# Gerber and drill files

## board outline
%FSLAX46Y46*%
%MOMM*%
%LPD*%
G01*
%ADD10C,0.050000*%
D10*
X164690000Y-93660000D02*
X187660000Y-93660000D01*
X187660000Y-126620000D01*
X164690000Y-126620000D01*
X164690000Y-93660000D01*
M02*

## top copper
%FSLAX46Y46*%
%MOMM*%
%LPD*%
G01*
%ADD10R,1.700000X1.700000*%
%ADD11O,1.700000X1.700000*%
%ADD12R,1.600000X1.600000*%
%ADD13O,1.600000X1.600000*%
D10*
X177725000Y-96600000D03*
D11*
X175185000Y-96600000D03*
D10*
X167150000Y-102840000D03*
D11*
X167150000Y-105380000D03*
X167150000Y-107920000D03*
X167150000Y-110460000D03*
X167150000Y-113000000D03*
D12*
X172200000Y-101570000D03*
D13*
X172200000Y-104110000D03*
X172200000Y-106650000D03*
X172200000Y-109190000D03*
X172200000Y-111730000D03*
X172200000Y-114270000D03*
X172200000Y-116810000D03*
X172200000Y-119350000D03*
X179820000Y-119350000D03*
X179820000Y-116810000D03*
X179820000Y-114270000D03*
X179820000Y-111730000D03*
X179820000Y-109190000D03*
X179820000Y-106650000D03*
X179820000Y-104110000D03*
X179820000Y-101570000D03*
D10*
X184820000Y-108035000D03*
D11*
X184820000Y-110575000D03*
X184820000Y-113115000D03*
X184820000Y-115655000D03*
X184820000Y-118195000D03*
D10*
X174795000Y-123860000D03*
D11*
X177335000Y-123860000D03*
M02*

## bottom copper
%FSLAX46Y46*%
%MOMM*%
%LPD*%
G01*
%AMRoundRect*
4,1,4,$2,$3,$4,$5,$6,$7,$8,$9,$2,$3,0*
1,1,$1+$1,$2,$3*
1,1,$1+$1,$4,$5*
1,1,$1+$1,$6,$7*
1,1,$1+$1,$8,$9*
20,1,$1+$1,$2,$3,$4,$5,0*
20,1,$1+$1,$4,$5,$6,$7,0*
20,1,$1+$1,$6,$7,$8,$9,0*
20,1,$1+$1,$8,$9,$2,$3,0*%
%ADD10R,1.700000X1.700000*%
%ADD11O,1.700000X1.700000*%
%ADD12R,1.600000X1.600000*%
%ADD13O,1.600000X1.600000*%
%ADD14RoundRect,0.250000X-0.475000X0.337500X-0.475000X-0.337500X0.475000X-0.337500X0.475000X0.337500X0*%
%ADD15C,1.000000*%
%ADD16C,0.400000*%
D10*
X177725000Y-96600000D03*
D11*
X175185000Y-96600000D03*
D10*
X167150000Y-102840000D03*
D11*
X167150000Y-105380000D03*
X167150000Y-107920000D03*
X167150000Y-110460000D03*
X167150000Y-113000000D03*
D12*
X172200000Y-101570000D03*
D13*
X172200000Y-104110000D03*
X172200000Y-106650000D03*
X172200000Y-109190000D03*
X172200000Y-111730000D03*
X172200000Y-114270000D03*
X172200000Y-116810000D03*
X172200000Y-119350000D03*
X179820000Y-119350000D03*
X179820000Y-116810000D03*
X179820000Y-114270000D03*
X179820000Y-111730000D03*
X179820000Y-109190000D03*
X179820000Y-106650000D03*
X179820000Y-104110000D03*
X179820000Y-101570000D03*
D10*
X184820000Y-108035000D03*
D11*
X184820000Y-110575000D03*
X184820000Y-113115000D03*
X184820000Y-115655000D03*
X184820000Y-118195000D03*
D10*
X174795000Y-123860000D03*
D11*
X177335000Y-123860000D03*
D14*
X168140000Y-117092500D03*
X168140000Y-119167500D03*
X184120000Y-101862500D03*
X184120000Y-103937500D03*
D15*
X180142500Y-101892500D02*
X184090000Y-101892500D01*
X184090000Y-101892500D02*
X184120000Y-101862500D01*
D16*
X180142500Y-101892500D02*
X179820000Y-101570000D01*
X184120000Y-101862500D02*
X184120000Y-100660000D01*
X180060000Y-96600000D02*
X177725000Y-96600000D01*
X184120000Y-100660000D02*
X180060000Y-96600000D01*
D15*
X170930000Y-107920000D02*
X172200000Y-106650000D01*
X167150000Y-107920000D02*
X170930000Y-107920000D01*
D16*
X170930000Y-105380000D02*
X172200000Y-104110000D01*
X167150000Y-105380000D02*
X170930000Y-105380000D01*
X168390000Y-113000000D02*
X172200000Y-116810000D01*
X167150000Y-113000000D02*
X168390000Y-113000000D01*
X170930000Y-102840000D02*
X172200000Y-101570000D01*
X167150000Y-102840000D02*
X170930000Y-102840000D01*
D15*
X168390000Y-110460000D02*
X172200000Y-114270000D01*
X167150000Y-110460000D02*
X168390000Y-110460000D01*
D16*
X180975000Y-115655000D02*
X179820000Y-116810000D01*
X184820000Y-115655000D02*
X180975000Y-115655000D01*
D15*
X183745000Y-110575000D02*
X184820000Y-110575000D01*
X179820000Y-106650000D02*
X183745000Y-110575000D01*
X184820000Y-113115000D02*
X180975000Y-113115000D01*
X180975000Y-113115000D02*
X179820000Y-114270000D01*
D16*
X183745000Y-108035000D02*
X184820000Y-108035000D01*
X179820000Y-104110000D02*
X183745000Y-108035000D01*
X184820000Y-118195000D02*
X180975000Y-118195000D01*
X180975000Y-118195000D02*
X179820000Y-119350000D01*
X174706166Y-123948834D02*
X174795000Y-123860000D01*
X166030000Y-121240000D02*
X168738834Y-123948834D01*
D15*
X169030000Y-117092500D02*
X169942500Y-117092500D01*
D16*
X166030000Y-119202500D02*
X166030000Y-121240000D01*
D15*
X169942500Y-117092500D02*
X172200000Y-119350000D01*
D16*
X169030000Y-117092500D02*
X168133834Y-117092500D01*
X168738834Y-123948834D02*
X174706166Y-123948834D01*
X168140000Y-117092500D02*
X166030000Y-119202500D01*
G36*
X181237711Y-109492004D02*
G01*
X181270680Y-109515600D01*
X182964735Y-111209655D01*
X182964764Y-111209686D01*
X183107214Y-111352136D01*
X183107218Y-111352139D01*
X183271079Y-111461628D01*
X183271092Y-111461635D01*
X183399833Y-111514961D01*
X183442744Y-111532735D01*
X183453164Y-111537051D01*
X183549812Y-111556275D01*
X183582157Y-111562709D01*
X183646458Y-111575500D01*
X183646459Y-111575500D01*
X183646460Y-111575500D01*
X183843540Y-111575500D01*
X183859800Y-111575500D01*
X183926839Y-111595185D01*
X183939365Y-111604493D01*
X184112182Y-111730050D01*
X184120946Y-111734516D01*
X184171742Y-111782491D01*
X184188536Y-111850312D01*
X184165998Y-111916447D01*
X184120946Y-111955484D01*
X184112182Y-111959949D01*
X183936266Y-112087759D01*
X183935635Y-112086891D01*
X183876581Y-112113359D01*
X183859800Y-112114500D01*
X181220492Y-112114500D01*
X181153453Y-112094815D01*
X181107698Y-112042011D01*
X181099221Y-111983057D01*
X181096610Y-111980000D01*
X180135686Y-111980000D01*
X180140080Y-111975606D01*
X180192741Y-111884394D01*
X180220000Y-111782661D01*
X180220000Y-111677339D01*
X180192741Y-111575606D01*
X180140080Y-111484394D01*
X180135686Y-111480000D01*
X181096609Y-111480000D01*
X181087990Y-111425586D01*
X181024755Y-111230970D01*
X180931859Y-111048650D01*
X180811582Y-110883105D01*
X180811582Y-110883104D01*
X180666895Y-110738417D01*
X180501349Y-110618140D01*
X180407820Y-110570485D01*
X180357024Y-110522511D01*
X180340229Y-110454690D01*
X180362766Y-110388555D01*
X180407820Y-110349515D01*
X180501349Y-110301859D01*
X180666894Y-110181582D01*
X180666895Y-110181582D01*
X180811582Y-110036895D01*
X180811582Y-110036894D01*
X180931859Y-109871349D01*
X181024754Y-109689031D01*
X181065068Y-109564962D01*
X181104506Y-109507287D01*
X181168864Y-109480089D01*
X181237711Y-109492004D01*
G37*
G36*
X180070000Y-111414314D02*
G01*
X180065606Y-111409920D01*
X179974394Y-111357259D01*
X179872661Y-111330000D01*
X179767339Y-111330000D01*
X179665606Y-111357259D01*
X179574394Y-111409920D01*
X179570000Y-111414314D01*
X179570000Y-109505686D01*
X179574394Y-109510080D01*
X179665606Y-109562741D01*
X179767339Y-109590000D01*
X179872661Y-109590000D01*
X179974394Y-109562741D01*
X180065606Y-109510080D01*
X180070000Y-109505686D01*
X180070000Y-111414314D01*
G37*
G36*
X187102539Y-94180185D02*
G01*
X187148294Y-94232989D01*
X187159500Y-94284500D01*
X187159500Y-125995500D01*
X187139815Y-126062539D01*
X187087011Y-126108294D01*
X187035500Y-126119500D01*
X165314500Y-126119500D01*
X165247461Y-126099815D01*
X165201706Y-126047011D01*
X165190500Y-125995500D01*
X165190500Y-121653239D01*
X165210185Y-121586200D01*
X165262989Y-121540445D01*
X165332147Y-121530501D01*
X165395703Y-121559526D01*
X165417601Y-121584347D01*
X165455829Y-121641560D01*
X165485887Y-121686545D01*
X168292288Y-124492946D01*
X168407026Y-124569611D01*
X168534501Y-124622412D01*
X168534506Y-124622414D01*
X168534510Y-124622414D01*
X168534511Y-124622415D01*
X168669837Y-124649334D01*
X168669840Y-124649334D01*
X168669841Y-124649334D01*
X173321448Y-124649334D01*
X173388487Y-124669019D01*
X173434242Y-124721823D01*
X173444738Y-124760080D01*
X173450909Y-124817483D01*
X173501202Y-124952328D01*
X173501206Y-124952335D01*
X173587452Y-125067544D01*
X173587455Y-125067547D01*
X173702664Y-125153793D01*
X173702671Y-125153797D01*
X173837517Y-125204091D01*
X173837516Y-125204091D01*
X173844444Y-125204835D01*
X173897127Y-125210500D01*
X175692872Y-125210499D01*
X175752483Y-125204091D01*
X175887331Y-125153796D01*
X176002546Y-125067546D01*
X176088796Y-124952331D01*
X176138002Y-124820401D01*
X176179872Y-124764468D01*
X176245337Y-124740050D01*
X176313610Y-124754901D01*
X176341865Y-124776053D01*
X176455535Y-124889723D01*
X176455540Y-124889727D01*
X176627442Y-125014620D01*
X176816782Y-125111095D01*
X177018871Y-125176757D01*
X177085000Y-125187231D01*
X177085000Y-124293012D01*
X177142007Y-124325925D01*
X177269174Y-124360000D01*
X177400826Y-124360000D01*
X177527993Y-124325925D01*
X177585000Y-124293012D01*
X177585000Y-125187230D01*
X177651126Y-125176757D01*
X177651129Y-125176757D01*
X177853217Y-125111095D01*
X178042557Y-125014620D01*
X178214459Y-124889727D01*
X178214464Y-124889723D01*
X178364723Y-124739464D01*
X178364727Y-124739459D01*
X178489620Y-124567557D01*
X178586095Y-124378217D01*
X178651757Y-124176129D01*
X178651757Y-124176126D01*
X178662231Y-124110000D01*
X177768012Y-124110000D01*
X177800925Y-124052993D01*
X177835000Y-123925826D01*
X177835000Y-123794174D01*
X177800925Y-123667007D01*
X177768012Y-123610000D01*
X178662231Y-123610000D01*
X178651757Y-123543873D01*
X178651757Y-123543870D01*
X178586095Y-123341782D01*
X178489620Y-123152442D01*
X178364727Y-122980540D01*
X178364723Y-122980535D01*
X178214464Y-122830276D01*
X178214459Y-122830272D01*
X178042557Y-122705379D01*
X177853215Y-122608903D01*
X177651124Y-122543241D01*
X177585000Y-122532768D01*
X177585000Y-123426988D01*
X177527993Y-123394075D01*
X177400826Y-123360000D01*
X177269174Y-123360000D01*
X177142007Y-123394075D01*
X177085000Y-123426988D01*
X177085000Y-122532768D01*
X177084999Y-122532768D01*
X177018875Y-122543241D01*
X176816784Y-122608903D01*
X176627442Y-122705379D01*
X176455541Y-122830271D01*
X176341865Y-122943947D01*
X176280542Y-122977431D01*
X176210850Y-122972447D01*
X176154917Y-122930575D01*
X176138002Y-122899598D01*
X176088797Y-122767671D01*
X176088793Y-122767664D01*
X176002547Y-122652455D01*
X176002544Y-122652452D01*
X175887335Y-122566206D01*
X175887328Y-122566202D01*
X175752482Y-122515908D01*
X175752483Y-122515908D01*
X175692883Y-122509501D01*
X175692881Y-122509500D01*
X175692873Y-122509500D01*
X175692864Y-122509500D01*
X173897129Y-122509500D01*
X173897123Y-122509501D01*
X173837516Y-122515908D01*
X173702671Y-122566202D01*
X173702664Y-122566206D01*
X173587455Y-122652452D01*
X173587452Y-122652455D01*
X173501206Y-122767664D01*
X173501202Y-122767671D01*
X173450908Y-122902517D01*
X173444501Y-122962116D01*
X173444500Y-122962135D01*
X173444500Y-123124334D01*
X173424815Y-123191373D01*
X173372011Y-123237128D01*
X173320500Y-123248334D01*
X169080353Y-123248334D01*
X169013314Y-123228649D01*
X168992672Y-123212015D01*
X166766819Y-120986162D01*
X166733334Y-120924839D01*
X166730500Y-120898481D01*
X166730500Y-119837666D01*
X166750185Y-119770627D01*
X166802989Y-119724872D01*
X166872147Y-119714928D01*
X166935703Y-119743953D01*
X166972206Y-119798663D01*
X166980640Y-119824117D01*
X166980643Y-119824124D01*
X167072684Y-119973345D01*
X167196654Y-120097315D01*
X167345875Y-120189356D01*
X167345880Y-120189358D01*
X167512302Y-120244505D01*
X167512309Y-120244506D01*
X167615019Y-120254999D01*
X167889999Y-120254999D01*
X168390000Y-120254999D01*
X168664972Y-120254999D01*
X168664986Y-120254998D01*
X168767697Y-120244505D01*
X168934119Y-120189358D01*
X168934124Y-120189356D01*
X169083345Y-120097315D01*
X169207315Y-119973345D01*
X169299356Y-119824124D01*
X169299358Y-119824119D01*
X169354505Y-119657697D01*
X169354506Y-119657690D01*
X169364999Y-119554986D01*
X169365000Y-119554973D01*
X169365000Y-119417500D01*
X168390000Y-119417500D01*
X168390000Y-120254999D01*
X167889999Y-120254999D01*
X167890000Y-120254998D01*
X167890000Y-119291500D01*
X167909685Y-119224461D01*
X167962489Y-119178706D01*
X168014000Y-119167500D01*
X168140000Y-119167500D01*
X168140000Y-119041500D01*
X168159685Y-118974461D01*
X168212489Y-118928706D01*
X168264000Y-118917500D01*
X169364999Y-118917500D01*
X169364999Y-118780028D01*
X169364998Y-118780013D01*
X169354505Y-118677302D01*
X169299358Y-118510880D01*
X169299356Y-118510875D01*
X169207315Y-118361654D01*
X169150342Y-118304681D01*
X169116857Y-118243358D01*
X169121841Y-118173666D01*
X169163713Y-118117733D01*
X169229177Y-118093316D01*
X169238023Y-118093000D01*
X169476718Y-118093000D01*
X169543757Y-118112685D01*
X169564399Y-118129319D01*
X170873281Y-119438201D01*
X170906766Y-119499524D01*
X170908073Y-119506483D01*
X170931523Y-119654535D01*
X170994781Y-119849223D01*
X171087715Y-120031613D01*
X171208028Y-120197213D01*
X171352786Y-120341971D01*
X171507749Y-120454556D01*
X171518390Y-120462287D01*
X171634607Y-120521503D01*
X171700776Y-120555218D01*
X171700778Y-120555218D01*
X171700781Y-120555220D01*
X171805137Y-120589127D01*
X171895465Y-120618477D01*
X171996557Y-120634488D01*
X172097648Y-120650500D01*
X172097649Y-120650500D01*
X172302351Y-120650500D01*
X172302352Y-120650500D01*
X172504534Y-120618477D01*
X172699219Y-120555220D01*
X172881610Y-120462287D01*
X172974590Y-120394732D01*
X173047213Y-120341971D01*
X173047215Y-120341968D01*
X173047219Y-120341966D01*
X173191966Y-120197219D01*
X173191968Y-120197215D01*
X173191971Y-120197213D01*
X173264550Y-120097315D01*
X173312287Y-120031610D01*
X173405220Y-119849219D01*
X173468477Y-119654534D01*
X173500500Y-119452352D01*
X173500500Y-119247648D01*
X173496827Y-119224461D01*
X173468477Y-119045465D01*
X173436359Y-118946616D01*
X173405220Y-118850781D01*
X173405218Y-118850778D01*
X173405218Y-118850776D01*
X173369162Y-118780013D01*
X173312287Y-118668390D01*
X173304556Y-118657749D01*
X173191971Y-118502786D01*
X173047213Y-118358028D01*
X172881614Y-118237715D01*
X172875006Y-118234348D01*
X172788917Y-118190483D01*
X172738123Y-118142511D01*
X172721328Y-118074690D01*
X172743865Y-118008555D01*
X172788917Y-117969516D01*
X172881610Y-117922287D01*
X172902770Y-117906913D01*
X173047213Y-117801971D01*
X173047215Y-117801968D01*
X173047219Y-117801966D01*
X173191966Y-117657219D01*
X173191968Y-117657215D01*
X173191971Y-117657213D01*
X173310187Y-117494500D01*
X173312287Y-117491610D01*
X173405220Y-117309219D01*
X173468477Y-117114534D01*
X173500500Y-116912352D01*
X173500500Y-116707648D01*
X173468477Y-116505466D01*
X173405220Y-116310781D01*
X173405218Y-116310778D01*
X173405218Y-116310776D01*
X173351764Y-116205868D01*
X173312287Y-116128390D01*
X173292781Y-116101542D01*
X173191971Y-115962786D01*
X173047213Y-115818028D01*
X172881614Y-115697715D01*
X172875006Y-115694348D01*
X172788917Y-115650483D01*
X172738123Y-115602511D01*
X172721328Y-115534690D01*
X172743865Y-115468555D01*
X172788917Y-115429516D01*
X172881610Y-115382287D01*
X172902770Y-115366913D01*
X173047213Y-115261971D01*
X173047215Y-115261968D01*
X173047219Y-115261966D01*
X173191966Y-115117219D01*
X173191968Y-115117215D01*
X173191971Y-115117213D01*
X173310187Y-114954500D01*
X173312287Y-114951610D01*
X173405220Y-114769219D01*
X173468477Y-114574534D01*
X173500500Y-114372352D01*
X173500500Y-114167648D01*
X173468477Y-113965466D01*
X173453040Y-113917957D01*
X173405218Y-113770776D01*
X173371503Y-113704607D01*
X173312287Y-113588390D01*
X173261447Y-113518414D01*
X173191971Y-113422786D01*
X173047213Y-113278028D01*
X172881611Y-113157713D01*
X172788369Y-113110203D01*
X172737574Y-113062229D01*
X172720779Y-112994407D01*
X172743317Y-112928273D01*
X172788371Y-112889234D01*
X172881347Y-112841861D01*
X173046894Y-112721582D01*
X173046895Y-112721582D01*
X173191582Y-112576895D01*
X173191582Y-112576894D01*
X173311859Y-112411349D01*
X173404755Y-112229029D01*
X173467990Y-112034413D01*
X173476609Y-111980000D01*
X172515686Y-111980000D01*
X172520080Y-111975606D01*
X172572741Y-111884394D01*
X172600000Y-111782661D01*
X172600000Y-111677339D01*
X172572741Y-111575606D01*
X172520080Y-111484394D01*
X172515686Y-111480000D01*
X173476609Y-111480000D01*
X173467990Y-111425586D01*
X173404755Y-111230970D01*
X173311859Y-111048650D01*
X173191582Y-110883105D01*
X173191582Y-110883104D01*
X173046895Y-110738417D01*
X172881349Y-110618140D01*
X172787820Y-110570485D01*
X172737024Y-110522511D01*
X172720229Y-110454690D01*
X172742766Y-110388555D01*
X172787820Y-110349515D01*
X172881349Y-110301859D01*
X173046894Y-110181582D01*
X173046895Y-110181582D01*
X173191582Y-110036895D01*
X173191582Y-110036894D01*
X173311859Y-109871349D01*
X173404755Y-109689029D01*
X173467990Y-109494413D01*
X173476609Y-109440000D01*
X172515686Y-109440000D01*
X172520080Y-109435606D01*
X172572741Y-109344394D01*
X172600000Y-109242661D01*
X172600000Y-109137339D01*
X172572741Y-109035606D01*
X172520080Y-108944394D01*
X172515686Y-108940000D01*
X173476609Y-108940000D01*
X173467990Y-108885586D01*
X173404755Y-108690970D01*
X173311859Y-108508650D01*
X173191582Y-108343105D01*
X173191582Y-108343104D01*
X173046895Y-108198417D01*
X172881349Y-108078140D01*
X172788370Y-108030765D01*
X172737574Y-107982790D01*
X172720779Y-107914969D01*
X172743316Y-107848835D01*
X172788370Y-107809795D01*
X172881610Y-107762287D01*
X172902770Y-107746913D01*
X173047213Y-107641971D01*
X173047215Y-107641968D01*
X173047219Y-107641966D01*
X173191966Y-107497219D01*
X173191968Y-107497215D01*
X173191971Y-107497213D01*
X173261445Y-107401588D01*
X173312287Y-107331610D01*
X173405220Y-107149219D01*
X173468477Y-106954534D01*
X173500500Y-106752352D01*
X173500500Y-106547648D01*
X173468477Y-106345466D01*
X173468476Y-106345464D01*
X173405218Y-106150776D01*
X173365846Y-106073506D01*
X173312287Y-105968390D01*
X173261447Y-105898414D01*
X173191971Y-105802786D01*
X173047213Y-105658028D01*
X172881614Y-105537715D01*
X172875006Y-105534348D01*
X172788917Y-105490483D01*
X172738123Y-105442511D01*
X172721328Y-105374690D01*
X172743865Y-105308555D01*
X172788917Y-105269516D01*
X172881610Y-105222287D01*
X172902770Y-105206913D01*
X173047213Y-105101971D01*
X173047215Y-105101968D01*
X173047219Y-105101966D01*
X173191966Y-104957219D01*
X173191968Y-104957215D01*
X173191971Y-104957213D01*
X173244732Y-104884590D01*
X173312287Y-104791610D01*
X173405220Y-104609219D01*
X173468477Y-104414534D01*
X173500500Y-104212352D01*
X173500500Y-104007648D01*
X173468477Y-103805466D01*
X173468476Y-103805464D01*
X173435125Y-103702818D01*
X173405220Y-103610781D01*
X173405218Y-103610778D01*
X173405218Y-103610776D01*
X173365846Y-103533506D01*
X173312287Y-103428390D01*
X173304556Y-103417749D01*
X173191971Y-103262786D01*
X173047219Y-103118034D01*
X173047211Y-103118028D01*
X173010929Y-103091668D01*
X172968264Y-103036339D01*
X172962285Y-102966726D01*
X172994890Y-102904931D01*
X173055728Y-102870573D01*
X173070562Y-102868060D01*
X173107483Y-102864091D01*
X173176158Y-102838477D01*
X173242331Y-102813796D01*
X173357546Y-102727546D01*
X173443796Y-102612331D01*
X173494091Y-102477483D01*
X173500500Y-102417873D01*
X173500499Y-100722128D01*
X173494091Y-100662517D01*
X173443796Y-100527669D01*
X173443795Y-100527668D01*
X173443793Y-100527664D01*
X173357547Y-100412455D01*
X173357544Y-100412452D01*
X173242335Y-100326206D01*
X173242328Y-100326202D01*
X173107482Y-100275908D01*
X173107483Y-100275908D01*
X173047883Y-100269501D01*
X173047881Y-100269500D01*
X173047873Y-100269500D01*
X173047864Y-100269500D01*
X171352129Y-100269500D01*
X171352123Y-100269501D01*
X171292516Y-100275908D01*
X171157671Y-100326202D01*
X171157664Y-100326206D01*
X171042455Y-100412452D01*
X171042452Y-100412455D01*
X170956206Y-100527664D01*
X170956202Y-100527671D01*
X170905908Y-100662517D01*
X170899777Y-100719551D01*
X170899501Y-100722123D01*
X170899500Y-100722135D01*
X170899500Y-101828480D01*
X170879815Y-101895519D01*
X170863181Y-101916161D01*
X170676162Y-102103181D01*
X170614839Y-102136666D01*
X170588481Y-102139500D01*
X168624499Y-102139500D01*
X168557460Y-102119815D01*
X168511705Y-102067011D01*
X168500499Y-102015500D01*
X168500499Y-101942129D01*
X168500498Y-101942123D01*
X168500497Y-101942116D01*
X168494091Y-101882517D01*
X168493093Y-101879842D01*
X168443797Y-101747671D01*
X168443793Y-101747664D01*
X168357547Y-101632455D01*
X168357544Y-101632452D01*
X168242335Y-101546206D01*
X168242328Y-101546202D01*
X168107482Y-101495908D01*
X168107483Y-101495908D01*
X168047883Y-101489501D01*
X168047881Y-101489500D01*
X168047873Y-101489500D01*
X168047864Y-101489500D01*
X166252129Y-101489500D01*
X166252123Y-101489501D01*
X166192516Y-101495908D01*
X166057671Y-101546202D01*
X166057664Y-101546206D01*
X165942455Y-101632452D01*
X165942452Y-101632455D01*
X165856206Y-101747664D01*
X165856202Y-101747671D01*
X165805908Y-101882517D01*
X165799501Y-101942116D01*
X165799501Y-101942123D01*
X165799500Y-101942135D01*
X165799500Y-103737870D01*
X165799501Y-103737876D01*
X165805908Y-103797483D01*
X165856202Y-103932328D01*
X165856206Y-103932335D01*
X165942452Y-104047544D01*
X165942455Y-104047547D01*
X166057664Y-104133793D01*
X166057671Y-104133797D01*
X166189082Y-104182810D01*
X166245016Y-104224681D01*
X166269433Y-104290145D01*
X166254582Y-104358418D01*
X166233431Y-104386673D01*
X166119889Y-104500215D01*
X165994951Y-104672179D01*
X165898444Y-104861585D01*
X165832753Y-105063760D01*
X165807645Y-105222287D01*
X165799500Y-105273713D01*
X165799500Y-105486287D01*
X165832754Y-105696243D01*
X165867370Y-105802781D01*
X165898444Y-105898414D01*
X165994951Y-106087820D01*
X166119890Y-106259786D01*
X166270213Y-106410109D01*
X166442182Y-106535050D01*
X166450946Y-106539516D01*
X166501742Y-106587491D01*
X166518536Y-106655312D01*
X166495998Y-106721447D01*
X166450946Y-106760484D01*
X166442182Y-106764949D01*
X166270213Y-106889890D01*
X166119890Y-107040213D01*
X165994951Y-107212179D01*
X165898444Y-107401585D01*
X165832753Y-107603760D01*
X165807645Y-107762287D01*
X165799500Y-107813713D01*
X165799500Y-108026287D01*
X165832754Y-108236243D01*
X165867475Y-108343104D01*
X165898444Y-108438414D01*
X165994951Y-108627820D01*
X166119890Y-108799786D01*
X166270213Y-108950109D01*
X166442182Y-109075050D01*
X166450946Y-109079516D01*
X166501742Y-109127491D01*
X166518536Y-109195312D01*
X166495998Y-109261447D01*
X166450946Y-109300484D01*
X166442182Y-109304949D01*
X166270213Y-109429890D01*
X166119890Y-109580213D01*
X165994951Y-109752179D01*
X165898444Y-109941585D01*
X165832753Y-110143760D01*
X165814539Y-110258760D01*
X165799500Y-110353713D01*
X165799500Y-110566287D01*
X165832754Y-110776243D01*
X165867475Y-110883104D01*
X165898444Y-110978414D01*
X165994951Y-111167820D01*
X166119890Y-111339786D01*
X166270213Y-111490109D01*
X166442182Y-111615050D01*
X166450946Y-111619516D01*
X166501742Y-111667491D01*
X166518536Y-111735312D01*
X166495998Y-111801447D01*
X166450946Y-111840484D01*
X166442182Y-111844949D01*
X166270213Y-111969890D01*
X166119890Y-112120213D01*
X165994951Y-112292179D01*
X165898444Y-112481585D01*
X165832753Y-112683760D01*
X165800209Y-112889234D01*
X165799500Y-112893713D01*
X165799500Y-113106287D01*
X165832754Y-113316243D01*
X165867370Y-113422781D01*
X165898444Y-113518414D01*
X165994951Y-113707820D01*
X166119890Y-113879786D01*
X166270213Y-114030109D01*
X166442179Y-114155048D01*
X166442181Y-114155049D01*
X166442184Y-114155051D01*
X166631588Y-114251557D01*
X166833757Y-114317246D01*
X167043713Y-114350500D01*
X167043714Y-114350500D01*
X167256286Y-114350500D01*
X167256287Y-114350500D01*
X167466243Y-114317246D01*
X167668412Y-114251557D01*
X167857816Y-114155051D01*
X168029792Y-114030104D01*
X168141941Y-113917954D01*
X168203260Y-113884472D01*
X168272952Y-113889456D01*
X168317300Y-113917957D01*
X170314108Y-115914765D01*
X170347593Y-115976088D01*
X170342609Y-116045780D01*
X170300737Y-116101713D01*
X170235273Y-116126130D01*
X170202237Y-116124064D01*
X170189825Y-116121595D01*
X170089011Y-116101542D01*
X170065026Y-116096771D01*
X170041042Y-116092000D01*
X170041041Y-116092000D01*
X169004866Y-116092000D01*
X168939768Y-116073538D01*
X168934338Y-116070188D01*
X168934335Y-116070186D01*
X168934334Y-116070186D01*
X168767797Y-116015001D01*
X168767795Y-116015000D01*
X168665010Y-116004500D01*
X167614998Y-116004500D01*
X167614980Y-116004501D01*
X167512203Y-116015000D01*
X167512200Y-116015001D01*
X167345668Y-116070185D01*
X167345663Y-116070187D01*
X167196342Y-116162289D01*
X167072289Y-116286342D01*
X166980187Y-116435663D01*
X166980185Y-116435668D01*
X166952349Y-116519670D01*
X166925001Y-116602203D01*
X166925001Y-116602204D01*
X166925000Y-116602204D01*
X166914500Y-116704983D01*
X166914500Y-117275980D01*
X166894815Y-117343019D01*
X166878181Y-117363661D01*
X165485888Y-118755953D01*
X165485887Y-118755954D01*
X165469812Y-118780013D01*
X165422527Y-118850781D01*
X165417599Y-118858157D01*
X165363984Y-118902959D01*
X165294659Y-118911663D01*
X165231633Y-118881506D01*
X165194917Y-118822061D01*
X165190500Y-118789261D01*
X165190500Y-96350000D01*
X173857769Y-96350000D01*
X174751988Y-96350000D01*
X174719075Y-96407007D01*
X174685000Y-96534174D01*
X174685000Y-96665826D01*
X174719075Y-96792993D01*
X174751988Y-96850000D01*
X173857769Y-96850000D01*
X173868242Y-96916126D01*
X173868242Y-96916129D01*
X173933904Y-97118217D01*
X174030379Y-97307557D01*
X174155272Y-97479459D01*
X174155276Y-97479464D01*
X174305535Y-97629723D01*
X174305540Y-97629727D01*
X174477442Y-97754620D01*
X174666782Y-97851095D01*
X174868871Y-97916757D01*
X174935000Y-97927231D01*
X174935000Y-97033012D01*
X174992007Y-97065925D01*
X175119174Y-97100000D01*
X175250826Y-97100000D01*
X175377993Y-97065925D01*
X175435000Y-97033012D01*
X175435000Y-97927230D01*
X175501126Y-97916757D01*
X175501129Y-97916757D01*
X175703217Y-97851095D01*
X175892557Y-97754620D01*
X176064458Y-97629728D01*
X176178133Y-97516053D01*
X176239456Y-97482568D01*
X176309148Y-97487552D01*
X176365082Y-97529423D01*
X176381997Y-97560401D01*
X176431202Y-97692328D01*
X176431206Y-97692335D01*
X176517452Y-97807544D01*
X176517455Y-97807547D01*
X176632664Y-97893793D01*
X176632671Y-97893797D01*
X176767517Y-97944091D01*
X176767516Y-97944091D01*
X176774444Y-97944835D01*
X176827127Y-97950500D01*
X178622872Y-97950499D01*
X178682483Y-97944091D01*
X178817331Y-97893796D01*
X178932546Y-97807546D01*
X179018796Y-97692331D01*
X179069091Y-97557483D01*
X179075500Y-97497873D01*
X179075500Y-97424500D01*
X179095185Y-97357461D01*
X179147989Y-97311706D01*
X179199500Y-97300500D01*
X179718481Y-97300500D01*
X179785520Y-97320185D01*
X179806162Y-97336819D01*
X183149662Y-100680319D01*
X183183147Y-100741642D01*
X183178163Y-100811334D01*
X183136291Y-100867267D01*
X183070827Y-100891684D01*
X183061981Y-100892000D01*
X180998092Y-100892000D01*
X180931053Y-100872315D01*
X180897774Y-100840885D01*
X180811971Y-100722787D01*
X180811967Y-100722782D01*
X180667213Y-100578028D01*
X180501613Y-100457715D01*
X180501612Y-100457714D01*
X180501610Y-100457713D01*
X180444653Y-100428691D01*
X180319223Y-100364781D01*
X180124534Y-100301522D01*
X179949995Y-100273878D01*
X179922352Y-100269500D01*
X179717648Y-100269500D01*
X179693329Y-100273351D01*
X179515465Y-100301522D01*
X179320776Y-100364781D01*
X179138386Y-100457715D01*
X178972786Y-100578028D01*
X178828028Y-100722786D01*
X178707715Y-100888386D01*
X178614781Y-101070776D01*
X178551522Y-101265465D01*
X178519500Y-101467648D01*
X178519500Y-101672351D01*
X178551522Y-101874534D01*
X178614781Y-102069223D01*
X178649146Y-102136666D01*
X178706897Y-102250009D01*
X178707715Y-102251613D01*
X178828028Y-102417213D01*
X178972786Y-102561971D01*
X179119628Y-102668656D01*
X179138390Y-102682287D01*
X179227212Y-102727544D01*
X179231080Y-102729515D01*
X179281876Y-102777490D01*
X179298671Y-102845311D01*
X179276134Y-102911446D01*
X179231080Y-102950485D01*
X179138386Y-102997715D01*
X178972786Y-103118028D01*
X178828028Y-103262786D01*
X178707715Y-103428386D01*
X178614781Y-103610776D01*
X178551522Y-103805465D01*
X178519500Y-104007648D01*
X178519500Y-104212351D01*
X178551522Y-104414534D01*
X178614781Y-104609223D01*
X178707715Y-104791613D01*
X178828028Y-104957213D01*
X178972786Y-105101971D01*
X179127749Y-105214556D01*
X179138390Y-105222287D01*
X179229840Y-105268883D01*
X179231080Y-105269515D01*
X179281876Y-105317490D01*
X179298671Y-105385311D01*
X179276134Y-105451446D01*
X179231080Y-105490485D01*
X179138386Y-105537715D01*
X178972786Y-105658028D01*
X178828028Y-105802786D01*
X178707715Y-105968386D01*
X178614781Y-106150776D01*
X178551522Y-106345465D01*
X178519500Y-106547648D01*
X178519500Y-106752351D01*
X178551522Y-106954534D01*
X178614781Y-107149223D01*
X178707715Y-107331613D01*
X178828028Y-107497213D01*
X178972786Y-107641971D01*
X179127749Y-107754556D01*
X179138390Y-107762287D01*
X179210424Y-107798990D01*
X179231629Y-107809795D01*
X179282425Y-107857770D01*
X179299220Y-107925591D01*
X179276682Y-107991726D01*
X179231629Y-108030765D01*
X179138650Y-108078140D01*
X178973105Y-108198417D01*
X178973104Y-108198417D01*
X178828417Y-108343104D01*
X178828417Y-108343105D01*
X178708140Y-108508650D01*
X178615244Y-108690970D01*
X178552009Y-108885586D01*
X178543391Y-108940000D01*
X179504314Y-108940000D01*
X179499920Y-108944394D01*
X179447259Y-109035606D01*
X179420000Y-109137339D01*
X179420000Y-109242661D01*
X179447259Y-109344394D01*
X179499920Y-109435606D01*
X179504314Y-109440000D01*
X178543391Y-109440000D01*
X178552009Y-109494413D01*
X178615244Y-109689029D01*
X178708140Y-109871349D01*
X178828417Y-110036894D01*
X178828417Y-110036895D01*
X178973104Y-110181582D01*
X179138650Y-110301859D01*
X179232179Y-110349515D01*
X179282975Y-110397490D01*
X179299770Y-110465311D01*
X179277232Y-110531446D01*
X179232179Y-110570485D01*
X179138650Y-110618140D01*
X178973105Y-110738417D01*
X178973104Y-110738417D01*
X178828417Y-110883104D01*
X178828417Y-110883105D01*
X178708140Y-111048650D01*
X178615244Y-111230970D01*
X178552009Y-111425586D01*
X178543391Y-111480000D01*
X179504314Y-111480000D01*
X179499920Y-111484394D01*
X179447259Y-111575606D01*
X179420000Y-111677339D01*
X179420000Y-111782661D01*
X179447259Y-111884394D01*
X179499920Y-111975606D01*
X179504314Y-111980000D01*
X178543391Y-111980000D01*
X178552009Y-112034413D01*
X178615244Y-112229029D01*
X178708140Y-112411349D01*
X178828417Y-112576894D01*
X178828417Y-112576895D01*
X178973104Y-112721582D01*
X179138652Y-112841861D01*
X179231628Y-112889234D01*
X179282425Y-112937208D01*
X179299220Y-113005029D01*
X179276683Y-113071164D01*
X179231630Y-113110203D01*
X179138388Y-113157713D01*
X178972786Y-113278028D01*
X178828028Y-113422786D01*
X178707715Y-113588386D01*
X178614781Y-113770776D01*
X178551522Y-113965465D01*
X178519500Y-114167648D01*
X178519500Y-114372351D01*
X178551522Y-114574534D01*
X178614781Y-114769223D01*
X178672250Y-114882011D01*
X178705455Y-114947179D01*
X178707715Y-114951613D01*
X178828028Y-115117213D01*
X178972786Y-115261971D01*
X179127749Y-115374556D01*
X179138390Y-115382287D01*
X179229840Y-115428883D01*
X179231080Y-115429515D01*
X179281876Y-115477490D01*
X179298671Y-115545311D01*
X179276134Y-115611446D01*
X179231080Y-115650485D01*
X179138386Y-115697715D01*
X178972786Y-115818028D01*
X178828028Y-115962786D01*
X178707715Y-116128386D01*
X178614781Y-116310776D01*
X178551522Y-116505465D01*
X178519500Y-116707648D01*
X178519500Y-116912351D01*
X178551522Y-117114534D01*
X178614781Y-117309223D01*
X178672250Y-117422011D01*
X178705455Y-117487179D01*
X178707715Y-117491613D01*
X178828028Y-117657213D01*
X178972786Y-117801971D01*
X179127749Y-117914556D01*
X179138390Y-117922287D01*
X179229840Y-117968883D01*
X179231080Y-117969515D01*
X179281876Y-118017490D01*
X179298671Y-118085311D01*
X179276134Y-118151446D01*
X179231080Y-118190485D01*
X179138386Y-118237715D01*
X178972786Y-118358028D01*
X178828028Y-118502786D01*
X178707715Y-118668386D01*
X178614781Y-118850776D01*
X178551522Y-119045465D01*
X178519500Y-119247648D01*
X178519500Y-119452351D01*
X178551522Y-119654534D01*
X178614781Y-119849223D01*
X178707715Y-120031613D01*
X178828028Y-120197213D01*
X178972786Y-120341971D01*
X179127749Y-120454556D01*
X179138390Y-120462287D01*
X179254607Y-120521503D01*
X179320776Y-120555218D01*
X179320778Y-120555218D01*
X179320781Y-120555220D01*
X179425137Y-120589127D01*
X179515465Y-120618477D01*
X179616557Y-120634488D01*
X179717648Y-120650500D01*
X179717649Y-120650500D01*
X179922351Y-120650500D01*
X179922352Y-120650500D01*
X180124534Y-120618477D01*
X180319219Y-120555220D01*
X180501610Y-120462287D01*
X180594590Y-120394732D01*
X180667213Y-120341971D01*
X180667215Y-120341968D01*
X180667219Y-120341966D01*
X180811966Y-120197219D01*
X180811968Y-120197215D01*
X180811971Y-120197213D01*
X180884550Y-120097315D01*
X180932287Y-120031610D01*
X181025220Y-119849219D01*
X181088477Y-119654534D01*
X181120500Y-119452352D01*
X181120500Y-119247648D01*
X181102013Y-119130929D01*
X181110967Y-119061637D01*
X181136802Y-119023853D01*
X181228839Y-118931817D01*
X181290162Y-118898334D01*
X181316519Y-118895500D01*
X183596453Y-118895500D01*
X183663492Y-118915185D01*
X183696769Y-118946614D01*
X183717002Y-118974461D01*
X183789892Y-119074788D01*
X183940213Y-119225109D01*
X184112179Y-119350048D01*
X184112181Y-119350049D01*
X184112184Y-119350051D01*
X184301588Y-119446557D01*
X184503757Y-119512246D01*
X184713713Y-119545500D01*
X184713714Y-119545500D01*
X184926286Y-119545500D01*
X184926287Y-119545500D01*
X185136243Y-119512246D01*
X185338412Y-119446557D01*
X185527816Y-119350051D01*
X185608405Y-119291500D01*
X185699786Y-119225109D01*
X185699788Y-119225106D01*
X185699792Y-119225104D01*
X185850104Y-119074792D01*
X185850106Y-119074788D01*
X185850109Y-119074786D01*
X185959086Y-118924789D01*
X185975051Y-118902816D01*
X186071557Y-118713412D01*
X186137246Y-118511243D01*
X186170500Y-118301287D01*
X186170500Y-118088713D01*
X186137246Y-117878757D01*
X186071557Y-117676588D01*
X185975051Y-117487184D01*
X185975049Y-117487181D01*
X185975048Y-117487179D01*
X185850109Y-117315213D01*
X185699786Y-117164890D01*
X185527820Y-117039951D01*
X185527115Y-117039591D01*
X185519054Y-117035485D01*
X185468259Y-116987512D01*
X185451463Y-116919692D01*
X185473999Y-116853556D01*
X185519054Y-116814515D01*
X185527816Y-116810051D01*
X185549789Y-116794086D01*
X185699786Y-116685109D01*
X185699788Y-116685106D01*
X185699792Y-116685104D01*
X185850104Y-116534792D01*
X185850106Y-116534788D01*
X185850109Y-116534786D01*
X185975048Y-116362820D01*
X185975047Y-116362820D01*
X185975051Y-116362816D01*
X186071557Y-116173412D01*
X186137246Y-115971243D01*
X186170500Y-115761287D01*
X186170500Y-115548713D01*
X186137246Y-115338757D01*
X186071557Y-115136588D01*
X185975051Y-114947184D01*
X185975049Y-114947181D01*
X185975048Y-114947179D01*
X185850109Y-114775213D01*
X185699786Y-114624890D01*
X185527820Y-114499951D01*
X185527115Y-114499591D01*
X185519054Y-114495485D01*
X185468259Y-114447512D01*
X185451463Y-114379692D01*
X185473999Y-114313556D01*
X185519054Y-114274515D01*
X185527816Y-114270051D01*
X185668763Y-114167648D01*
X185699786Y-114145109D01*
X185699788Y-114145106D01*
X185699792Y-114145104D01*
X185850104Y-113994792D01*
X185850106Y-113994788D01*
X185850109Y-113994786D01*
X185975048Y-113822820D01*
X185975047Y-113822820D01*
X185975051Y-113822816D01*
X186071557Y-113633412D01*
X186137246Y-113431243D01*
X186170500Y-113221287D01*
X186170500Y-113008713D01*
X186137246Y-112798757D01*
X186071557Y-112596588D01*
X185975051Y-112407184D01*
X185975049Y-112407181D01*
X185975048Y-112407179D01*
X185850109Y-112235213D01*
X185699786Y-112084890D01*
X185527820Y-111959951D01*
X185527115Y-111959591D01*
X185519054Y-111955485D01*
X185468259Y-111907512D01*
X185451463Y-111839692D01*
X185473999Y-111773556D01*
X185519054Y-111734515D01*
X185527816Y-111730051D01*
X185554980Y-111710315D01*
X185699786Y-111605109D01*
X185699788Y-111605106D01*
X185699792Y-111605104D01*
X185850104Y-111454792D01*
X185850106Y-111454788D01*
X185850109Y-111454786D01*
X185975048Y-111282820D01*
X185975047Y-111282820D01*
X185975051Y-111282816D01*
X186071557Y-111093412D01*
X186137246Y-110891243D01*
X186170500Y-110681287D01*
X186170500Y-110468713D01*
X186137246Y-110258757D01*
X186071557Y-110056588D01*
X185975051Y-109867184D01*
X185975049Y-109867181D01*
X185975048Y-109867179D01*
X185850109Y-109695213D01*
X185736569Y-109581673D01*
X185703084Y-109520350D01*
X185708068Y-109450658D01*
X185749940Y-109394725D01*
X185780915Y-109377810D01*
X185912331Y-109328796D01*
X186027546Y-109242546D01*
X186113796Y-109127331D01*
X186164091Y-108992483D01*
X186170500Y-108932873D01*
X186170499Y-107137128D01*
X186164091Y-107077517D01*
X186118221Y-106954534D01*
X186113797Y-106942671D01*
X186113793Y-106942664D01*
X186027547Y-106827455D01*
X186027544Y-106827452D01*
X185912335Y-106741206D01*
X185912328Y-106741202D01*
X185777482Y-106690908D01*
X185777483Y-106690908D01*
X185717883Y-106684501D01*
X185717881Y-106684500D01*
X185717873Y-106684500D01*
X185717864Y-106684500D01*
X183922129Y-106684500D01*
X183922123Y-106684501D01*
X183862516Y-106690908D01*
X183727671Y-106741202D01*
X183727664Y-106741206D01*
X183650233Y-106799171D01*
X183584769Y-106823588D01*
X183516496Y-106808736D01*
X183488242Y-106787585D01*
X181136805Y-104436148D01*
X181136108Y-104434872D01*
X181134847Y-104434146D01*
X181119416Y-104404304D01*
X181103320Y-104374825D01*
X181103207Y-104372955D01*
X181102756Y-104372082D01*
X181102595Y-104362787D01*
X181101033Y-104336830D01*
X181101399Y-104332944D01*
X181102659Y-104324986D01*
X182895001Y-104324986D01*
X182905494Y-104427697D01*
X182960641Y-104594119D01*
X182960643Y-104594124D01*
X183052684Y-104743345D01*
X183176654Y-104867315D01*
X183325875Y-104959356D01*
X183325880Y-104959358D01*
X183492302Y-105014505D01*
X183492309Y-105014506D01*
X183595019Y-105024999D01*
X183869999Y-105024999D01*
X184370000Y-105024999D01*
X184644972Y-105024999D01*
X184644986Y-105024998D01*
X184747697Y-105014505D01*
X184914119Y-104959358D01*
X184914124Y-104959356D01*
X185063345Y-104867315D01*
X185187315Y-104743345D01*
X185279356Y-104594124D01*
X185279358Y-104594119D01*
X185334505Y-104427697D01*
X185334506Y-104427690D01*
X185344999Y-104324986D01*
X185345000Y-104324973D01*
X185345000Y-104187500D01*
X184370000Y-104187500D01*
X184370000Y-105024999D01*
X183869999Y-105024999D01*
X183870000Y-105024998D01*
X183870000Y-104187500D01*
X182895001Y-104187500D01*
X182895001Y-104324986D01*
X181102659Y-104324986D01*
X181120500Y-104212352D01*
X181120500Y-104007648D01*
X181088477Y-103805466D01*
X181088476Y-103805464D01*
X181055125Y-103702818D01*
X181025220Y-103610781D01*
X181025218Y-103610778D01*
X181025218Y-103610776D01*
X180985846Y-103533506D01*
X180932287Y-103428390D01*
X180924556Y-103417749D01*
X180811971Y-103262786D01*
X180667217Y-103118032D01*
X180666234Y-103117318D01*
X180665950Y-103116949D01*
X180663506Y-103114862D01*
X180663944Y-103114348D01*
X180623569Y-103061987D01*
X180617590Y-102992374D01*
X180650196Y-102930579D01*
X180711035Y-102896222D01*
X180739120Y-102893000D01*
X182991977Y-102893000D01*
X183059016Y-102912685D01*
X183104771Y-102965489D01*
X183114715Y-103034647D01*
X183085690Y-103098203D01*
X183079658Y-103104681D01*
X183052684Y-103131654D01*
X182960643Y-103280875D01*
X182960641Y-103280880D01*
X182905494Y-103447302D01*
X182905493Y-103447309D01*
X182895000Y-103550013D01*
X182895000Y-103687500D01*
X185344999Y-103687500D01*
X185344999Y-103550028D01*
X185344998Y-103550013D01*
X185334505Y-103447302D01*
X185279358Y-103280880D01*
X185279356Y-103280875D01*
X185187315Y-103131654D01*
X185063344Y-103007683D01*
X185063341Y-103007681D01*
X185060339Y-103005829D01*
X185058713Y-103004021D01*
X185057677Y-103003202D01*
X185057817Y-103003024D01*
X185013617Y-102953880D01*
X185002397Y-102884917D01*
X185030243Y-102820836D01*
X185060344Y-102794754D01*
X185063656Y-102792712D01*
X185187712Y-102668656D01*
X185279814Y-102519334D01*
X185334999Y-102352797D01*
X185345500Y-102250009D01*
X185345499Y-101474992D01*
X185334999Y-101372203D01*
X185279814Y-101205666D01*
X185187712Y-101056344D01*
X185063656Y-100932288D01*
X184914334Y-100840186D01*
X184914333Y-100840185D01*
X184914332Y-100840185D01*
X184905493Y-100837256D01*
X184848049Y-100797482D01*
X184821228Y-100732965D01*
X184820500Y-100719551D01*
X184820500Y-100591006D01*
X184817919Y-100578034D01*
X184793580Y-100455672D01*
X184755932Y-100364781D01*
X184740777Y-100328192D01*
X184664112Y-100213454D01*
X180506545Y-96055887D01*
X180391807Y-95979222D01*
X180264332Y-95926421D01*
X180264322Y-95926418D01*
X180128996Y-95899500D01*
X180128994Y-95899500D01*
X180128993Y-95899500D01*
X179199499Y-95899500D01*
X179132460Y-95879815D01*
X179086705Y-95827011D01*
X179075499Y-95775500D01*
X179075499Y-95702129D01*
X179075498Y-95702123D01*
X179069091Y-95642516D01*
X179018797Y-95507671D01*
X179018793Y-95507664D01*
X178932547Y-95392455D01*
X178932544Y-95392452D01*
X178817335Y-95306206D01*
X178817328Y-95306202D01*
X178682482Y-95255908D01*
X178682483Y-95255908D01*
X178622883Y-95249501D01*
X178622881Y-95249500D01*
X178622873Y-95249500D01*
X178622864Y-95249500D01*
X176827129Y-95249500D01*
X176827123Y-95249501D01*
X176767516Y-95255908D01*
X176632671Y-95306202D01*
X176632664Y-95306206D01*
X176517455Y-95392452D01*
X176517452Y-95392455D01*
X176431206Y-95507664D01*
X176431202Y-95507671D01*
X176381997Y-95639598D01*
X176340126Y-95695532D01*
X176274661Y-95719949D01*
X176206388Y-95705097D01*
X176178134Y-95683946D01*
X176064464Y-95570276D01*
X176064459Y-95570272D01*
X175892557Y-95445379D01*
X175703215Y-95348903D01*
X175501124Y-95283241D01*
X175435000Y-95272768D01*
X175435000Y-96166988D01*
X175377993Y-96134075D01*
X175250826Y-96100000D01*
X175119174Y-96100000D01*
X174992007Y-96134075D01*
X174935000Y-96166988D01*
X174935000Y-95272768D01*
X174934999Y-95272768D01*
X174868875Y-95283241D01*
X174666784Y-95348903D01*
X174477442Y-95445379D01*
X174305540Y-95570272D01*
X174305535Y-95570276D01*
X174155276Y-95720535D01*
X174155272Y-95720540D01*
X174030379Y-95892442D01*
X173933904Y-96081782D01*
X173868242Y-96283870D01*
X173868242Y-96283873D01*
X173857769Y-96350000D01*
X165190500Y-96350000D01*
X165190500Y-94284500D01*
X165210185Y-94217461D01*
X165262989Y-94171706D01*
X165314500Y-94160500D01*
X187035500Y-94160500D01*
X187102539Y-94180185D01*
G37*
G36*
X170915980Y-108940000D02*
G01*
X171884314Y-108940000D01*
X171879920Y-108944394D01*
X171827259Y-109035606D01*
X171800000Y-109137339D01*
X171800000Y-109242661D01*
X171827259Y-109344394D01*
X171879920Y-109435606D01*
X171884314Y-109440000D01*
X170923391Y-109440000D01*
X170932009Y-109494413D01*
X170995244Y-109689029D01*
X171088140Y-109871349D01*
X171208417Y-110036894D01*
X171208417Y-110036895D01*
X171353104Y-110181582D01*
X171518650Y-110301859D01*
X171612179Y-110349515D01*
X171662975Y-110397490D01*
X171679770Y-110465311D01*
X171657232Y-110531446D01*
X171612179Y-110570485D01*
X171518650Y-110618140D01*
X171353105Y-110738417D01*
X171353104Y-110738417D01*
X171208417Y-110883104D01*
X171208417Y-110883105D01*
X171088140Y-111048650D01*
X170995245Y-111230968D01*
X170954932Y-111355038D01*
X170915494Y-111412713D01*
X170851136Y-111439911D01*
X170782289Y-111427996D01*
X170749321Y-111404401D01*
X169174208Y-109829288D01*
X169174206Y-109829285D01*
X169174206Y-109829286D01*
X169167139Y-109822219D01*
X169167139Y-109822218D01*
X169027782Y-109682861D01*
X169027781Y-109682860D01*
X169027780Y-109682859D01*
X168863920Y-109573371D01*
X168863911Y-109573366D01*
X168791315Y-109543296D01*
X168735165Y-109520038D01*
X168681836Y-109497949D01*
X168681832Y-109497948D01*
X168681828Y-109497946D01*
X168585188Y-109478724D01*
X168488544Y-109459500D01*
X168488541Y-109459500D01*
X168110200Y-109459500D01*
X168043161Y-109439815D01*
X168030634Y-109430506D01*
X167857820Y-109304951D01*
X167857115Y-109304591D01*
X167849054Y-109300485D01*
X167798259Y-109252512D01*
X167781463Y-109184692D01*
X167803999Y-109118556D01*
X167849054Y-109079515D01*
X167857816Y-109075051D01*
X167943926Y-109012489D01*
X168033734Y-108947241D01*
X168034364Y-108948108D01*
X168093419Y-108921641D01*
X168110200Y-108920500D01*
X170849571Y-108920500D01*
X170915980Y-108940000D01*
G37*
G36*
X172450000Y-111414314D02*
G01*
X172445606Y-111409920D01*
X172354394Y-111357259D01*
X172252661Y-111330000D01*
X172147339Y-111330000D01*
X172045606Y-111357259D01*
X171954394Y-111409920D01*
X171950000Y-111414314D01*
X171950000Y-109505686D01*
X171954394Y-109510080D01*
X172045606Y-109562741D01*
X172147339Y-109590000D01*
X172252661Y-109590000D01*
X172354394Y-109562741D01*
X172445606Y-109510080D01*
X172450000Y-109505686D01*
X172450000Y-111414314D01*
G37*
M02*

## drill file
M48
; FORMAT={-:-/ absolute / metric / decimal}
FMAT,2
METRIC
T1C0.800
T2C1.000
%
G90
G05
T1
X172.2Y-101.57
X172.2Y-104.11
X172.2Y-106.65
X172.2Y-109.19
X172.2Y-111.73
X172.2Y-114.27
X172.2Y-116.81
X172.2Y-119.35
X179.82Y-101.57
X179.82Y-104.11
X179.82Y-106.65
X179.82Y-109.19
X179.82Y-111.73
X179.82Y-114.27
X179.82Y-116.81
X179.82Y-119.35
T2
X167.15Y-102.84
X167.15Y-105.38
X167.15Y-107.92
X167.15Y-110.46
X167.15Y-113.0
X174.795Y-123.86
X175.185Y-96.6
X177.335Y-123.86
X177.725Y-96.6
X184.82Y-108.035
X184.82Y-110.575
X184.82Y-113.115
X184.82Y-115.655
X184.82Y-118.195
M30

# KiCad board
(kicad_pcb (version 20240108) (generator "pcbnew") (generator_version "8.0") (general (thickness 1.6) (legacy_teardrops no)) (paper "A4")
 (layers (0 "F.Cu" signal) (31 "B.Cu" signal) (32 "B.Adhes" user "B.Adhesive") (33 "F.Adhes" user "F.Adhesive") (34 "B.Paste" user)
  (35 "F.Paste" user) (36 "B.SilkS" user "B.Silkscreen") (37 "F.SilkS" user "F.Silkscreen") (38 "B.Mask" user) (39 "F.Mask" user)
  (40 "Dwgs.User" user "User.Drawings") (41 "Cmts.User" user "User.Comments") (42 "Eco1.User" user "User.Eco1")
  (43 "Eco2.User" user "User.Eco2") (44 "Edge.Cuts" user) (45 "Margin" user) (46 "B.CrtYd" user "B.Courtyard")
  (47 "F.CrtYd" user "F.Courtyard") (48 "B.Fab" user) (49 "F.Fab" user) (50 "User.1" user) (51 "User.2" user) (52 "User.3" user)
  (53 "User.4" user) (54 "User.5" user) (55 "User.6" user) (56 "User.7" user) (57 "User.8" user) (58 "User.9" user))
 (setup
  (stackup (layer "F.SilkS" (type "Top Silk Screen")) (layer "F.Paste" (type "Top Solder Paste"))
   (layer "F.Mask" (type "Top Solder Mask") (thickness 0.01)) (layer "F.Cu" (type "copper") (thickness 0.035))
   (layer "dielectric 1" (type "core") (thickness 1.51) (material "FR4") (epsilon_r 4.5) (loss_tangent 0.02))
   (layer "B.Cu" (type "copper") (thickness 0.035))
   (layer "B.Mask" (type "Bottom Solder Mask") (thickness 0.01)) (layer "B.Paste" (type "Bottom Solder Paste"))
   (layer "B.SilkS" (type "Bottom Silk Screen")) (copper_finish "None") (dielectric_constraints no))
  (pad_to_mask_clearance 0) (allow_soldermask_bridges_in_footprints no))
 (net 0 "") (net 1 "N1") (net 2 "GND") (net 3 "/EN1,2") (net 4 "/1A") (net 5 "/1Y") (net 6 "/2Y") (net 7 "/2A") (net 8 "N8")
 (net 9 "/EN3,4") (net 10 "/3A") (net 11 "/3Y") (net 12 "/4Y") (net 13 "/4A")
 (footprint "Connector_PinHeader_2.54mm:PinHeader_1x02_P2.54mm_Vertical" (layer "F.Cu") (at 177.725 96.6 -90)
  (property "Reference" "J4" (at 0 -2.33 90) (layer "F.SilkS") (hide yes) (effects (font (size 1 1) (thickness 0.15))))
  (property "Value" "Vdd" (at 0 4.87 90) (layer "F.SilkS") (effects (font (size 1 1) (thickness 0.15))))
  (pad "1" thru_hole rect (at 0 0 270) (size 1.7 1.7) (drill 1) (layers "*.Cu" "*.Mask") (remove_unused_layers no) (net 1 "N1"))
  (pad "2" thru_hole oval (at 0 2.54 270) (size 1.7 1.7) (drill 1) (layers "*.Cu" "*.Mask") (remove_unused_layers no) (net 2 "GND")))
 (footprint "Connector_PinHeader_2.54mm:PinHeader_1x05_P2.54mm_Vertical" (layer "F.Cu") (at 167.15 102.84)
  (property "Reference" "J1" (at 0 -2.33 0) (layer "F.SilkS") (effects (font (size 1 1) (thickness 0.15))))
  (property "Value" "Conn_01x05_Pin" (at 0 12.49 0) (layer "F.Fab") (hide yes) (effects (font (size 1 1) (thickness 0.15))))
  (pad "1" thru_hole rect (at 0 0) (size 1.7 1.7) (drill 1) (layers "*.Cu" "*.Mask") (remove_unused_layers no) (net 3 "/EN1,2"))
  (pad "2" thru_hole oval (at 0 2.54) (size 1.7 1.7) (drill 1) (layers "*.Cu" "*.Mask") (remove_unused_layers no) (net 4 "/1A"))
  (pad "3" thru_hole oval (at 0 5.08) (size 1.7 1.7) (drill 1) (layers "*.Cu" "*.Mask") (remove_unused_layers no) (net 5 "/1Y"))
  (pad "4" thru_hole oval (at 0 7.62) (size 1.7 1.7) (drill 1) (layers "*.Cu" "*.Mask") (remove_unused_layers no) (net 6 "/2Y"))
  (pad "5" thru_hole oval (at 0 10.16) (size 1.7 1.7) (drill 1) (layers "*.Cu" "*.Mask") (remove_unused_layers no) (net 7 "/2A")))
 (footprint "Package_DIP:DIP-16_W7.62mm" (layer "F.Cu") (at 172.2 101.57)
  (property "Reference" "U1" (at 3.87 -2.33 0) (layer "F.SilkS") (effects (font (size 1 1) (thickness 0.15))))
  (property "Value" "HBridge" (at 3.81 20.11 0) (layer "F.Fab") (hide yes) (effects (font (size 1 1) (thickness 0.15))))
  (pad "1" thru_hole rect (at 0 0) (size 1.6 1.6) (drill 0.8) (layers "*.Cu" "*.Mask") (remove_unused_layers no) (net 3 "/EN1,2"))
  (pad "2" thru_hole oval (at 0 2.54) (size 1.6 1.6) (drill 0.8) (layers "*.Cu" "*.Mask") (remove_unused_layers no) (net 4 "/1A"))
  (pad "3" thru_hole oval (at 0 5.08) (size 1.6 1.6) (drill 0.8) (layers "*.Cu" "*.Mask") (remove_unused_layers no) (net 5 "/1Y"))
  (pad "4" thru_hole oval (at 0 7.62) (size 1.6 1.6) (drill 0.8) (layers "*.Cu" "*.Mask") (remove_unused_layers no) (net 2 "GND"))
  (pad "5" thru_hole oval (at 0 10.16) (size 1.6 1.6) (drill 0.8) (layers "*.Cu" "*.Mask") (remove_unused_layers no) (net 2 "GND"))
  (pad "6" thru_hole oval (at 0 12.7) (size 1.6 1.6) (drill 0.8) (layers "*.Cu" "*.Mask") (remove_unused_layers no) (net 6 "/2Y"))
  (pad "7" thru_hole oval (at 0 15.24) (size 1.6 1.6) (drill 0.8) (layers "*.Cu" "*.Mask") (remove_unused_layers no) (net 7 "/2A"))
  (pad "8" thru_hole oval (at 0 17.78) (size 1.6 1.6) (drill 0.8) (layers "*.Cu" "*.Mask") (remove_unused_layers no) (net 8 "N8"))
  (pad "9" thru_hole oval (at 7.62 17.78) (size 1.6 1.6) (drill 0.8) (layers "*.Cu" "*.Mask") (remove_unused_layers no) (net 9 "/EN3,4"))
  (pad "10" thru_hole oval (at 7.62 15.24) (size 1.6 1.6) (drill 0.8) (layers "*.Cu" "*.Mask") (remove_unused_layers no) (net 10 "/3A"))
  (pad "11" thru_hole oval (at 7.62 12.7) (size 1.6 1.6) (drill 0.8) (layers "*.Cu" "*.Mask") (remove_unused_layers no) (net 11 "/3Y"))
  (pad "12" thru_hole oval (at 7.62 10.16) (size 1.6 1.6) (drill 0.8) (layers "*.Cu" "*.Mask") (remove_unused_layers no) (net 2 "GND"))
  (pad "13" thru_hole oval (at 7.62 7.62) (size 1.6 1.6) (drill 0.8) (layers "*.Cu" "*.Mask") (remove_unused_layers no) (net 2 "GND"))
  (pad "14" thru_hole oval (at 7.62 5.08) (size 1.6 1.6) (drill 0.8) (layers "*.Cu" "*.Mask") (remove_unused_layers no) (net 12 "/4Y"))
  (pad "15" thru_hole oval (at 7.62 2.54) (size 1.6 1.6) (drill 0.8) (layers "*.Cu" "*.Mask") (remove_unused_layers no) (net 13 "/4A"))
  (pad "16" thru_hole oval (at 7.62 0) (size 1.6 1.6) (drill 0.8) (layers "*.Cu" "*.Mask") (remove_unused_layers no) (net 1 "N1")))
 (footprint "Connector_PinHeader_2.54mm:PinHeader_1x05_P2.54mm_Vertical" (layer "F.Cu") (at 184.82 108.035)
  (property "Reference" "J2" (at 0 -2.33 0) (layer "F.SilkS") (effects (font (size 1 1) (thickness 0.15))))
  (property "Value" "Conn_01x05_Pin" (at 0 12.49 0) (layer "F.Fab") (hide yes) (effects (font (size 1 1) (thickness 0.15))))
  (pad "1" thru_hole rect (at 0 0) (size 1.7 1.7) (drill 1) (layers "*.Cu" "*.Mask") (remove_unused_layers no) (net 13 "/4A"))
  (pad "2" thru_hole oval (at 0 2.54) (size 1.7 1.7) (drill 1) (layers "*.Cu" "*.Mask") (remove_unused_layers no) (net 12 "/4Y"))
  (pad "3" thru_hole oval (at 0 5.08) (size 1.7 1.7) (drill 1) (layers "*.Cu" "*.Mask") (remove_unused_layers no) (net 11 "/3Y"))
  (pad "4" thru_hole oval (at 0 7.62) (size 1.7 1.7) (drill 1) (layers "*.Cu" "*.Mask") (remove_unused_layers no) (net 10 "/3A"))
  (pad "5" thru_hole oval (at 0 10.16) (size 1.7 1.7) (drill 1) (layers "*.Cu" "*.Mask") (remove_unused_layers no) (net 9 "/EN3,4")))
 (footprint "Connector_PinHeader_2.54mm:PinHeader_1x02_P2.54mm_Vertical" (layer "F.Cu") (at 174.795 123.86 90)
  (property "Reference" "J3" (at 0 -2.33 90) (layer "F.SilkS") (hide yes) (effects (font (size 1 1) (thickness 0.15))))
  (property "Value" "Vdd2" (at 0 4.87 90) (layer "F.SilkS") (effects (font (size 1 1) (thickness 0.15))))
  (pad "1" thru_hole rect (at 0 0 90) (size 1.7 1.7) (drill 1) (layers "*.Cu" "*.Mask") (remove_unused_layers no) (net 8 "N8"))
  (pad "2" thru_hole oval (at 0 2.54 90) (size 1.7 1.7) (drill 1) (layers "*.Cu" "*.Mask") (remove_unused_layers no) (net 2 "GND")))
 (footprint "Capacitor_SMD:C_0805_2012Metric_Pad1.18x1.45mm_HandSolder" (layer "B.Cu") (at 168.14 118.13 -90)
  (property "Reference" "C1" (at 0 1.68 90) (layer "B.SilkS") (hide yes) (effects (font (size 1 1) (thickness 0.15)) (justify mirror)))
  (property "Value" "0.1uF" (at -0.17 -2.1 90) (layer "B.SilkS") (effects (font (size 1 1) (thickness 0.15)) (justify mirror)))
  (pad "1" smd roundrect (at -1.0375 0 270) (size 1.175 1.45) (layers "B.Cu" "B.Paste" "B.Mask") (roundrect_rratio 0.212766) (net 8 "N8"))
  (pad "2" smd roundrect (at 1.0375 0 270) (size 1.175 1.45) (layers "B.Cu" "B.Paste" "B.Mask") (roundrect_rratio 0.212766) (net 2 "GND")))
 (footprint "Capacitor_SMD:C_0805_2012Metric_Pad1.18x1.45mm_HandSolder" (layer "B.Cu") (at 184.12 102.9 -90)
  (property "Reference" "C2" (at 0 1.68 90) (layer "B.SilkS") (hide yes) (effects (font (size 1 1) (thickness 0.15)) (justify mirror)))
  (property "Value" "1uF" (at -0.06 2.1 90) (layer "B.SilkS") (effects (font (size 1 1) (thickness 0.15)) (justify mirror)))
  (pad "1" smd roundrect (at -1.0375 0 270) (size 1.175 1.45) (layers "B.Cu" "B.Paste" "B.Mask") (roundrect_rratio 0.212766) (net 1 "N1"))
  (pad "2" smd roundrect (at 1.0375 0 270) (size 1.175 1.45) (layers "B.Cu" "B.Paste" "B.Mask") (roundrect_rratio 0.212766) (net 2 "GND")))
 (gr_rect (start 164.69 93.66) (end 187.66 126.62) (stroke (width 0.05) (type default)) (fill none) (layer "Edge.Cuts"))
 (segment (start 180.1425 101.8925) (end 184.09 101.8925) (width 1) (layer "B.Cu") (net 1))
 (segment (start 184.09 101.8925) (end 184.12 101.8625) (width 1) (layer "B.Cu") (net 1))
 (segment (start 180.1425 101.8925) (end 179.82 101.57) (width 0.4) (layer "B.Cu") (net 1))
 (segment (start 184.12 101.8625) (end 184.12 100.66) (width 0.4) (layer "B.Cu") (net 1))
 (segment (start 180.06 96.6) (end 177.725 96.6) (width 0.4) (layer "B.Cu") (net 1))
 (segment (start 184.12 100.66) (end 180.06 96.6) (width 0.4) (layer "B.Cu") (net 1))
 (segment (start 170.93 107.92) (end 172.2 106.65) (width 1) (layer "B.Cu") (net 5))
 (segment (start 167.15 107.92) (end 170.93 107.92) (width 1) (layer "B.Cu") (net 5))
 (segment (start 170.93 105.38) (end 172.2 104.11) (width 0.4) (layer "B.Cu") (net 4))
 (segment (start 167.15 105.38) (end 170.93 105.38) (width 0.4) (layer "B.Cu") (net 4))
 (segment (start 168.39 113) (end 172.2 116.81) (width 0.4) (layer "B.Cu") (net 7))
 (segment (start 167.15 113) (end 168.39 113) (width 0.4) (layer "B.Cu") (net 7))
 (segment (start 170.93 102.84) (end 172.2 101.57) (width 0.4) (layer "B.Cu") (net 3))
 (segment (start 167.15 102.84) (end 170.93 102.84) (width 0.4) (layer "B.Cu") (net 3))
 (segment (start 168.39 110.46) (end 172.2 114.27) (width 1) (layer "B.Cu") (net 6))
 (segment (start 167.15 110.46) (end 168.39 110.46) (width 1) (layer "B.Cu") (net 6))
 (segment (start 180.975 115.655) (end 179.82 116.81) (width 0.4) (layer "B.Cu") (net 10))
 (segment (start 184.82 115.655) (end 180.975 115.655) (width 0.4) (layer "B.Cu") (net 10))
 (segment (start 183.745 110.575) (end 184.82 110.575) (width 1) (layer "B.Cu") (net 12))
 (segment (start 179.82 106.65) (end 183.745 110.575) (width 1) (layer "B.Cu") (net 12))
 (segment (start 184.82 113.115) (end 180.975 113.115) (width 1) (layer "B.Cu") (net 11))
 (segment (start 180.975 113.115) (end 179.82 114.27) (width 1) (layer "B.Cu") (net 11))
 (segment (start 183.745 108.035) (end 184.82 108.035) (width 0.4) (layer "B.Cu") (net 13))
 (segment (start 179.82 104.11) (end 183.745 108.035) (width 0.4) (layer "B.Cu") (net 13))
 (segment (start 184.82 118.195) (end 180.975 118.195) (width 0.4) (layer "B.Cu") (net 9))
 (segment (start 180.975 118.195) (end 179.82 119.35) (width 0.4) (layer "B.Cu") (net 9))
 (segment (start 174.706166 123.948834) (end 174.795 123.86) (width 0.4) (layer "B.Cu") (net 8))
 (segment (start 166.03 121.24) (end 168.738834 123.948834) (width 0.4) (layer "B.Cu") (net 8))
 (segment (start 169.03 117.0925) (end 169.9425 117.0925) (width 1) (layer "B.Cu") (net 8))
 (segment (start 166.03 119.2025) (end 166.03 121.24) (width 0.4) (layer "B.Cu") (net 8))
 (segment (start 169.9425 117.0925) (end 172.2 119.35) (width 1) (layer "B.Cu") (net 8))
 (segment (start 169.03 117.0925) (end 168.133834 117.0925) (width 0.4) (layer "B.Cu") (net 8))
 (segment (start 168.738834 123.948834) (end 174.706166 123.948834) (width 0.4) (layer "B.Cu") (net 8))
 (segment (start 168.14 117.0925) (end 166.03 119.2025) (width 0.4) (layer "B.Cu") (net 8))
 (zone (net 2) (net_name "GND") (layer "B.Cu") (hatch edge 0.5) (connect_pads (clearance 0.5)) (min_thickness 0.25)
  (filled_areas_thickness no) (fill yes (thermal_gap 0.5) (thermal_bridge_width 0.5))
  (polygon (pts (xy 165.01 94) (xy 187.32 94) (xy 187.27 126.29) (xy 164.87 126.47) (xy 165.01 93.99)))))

